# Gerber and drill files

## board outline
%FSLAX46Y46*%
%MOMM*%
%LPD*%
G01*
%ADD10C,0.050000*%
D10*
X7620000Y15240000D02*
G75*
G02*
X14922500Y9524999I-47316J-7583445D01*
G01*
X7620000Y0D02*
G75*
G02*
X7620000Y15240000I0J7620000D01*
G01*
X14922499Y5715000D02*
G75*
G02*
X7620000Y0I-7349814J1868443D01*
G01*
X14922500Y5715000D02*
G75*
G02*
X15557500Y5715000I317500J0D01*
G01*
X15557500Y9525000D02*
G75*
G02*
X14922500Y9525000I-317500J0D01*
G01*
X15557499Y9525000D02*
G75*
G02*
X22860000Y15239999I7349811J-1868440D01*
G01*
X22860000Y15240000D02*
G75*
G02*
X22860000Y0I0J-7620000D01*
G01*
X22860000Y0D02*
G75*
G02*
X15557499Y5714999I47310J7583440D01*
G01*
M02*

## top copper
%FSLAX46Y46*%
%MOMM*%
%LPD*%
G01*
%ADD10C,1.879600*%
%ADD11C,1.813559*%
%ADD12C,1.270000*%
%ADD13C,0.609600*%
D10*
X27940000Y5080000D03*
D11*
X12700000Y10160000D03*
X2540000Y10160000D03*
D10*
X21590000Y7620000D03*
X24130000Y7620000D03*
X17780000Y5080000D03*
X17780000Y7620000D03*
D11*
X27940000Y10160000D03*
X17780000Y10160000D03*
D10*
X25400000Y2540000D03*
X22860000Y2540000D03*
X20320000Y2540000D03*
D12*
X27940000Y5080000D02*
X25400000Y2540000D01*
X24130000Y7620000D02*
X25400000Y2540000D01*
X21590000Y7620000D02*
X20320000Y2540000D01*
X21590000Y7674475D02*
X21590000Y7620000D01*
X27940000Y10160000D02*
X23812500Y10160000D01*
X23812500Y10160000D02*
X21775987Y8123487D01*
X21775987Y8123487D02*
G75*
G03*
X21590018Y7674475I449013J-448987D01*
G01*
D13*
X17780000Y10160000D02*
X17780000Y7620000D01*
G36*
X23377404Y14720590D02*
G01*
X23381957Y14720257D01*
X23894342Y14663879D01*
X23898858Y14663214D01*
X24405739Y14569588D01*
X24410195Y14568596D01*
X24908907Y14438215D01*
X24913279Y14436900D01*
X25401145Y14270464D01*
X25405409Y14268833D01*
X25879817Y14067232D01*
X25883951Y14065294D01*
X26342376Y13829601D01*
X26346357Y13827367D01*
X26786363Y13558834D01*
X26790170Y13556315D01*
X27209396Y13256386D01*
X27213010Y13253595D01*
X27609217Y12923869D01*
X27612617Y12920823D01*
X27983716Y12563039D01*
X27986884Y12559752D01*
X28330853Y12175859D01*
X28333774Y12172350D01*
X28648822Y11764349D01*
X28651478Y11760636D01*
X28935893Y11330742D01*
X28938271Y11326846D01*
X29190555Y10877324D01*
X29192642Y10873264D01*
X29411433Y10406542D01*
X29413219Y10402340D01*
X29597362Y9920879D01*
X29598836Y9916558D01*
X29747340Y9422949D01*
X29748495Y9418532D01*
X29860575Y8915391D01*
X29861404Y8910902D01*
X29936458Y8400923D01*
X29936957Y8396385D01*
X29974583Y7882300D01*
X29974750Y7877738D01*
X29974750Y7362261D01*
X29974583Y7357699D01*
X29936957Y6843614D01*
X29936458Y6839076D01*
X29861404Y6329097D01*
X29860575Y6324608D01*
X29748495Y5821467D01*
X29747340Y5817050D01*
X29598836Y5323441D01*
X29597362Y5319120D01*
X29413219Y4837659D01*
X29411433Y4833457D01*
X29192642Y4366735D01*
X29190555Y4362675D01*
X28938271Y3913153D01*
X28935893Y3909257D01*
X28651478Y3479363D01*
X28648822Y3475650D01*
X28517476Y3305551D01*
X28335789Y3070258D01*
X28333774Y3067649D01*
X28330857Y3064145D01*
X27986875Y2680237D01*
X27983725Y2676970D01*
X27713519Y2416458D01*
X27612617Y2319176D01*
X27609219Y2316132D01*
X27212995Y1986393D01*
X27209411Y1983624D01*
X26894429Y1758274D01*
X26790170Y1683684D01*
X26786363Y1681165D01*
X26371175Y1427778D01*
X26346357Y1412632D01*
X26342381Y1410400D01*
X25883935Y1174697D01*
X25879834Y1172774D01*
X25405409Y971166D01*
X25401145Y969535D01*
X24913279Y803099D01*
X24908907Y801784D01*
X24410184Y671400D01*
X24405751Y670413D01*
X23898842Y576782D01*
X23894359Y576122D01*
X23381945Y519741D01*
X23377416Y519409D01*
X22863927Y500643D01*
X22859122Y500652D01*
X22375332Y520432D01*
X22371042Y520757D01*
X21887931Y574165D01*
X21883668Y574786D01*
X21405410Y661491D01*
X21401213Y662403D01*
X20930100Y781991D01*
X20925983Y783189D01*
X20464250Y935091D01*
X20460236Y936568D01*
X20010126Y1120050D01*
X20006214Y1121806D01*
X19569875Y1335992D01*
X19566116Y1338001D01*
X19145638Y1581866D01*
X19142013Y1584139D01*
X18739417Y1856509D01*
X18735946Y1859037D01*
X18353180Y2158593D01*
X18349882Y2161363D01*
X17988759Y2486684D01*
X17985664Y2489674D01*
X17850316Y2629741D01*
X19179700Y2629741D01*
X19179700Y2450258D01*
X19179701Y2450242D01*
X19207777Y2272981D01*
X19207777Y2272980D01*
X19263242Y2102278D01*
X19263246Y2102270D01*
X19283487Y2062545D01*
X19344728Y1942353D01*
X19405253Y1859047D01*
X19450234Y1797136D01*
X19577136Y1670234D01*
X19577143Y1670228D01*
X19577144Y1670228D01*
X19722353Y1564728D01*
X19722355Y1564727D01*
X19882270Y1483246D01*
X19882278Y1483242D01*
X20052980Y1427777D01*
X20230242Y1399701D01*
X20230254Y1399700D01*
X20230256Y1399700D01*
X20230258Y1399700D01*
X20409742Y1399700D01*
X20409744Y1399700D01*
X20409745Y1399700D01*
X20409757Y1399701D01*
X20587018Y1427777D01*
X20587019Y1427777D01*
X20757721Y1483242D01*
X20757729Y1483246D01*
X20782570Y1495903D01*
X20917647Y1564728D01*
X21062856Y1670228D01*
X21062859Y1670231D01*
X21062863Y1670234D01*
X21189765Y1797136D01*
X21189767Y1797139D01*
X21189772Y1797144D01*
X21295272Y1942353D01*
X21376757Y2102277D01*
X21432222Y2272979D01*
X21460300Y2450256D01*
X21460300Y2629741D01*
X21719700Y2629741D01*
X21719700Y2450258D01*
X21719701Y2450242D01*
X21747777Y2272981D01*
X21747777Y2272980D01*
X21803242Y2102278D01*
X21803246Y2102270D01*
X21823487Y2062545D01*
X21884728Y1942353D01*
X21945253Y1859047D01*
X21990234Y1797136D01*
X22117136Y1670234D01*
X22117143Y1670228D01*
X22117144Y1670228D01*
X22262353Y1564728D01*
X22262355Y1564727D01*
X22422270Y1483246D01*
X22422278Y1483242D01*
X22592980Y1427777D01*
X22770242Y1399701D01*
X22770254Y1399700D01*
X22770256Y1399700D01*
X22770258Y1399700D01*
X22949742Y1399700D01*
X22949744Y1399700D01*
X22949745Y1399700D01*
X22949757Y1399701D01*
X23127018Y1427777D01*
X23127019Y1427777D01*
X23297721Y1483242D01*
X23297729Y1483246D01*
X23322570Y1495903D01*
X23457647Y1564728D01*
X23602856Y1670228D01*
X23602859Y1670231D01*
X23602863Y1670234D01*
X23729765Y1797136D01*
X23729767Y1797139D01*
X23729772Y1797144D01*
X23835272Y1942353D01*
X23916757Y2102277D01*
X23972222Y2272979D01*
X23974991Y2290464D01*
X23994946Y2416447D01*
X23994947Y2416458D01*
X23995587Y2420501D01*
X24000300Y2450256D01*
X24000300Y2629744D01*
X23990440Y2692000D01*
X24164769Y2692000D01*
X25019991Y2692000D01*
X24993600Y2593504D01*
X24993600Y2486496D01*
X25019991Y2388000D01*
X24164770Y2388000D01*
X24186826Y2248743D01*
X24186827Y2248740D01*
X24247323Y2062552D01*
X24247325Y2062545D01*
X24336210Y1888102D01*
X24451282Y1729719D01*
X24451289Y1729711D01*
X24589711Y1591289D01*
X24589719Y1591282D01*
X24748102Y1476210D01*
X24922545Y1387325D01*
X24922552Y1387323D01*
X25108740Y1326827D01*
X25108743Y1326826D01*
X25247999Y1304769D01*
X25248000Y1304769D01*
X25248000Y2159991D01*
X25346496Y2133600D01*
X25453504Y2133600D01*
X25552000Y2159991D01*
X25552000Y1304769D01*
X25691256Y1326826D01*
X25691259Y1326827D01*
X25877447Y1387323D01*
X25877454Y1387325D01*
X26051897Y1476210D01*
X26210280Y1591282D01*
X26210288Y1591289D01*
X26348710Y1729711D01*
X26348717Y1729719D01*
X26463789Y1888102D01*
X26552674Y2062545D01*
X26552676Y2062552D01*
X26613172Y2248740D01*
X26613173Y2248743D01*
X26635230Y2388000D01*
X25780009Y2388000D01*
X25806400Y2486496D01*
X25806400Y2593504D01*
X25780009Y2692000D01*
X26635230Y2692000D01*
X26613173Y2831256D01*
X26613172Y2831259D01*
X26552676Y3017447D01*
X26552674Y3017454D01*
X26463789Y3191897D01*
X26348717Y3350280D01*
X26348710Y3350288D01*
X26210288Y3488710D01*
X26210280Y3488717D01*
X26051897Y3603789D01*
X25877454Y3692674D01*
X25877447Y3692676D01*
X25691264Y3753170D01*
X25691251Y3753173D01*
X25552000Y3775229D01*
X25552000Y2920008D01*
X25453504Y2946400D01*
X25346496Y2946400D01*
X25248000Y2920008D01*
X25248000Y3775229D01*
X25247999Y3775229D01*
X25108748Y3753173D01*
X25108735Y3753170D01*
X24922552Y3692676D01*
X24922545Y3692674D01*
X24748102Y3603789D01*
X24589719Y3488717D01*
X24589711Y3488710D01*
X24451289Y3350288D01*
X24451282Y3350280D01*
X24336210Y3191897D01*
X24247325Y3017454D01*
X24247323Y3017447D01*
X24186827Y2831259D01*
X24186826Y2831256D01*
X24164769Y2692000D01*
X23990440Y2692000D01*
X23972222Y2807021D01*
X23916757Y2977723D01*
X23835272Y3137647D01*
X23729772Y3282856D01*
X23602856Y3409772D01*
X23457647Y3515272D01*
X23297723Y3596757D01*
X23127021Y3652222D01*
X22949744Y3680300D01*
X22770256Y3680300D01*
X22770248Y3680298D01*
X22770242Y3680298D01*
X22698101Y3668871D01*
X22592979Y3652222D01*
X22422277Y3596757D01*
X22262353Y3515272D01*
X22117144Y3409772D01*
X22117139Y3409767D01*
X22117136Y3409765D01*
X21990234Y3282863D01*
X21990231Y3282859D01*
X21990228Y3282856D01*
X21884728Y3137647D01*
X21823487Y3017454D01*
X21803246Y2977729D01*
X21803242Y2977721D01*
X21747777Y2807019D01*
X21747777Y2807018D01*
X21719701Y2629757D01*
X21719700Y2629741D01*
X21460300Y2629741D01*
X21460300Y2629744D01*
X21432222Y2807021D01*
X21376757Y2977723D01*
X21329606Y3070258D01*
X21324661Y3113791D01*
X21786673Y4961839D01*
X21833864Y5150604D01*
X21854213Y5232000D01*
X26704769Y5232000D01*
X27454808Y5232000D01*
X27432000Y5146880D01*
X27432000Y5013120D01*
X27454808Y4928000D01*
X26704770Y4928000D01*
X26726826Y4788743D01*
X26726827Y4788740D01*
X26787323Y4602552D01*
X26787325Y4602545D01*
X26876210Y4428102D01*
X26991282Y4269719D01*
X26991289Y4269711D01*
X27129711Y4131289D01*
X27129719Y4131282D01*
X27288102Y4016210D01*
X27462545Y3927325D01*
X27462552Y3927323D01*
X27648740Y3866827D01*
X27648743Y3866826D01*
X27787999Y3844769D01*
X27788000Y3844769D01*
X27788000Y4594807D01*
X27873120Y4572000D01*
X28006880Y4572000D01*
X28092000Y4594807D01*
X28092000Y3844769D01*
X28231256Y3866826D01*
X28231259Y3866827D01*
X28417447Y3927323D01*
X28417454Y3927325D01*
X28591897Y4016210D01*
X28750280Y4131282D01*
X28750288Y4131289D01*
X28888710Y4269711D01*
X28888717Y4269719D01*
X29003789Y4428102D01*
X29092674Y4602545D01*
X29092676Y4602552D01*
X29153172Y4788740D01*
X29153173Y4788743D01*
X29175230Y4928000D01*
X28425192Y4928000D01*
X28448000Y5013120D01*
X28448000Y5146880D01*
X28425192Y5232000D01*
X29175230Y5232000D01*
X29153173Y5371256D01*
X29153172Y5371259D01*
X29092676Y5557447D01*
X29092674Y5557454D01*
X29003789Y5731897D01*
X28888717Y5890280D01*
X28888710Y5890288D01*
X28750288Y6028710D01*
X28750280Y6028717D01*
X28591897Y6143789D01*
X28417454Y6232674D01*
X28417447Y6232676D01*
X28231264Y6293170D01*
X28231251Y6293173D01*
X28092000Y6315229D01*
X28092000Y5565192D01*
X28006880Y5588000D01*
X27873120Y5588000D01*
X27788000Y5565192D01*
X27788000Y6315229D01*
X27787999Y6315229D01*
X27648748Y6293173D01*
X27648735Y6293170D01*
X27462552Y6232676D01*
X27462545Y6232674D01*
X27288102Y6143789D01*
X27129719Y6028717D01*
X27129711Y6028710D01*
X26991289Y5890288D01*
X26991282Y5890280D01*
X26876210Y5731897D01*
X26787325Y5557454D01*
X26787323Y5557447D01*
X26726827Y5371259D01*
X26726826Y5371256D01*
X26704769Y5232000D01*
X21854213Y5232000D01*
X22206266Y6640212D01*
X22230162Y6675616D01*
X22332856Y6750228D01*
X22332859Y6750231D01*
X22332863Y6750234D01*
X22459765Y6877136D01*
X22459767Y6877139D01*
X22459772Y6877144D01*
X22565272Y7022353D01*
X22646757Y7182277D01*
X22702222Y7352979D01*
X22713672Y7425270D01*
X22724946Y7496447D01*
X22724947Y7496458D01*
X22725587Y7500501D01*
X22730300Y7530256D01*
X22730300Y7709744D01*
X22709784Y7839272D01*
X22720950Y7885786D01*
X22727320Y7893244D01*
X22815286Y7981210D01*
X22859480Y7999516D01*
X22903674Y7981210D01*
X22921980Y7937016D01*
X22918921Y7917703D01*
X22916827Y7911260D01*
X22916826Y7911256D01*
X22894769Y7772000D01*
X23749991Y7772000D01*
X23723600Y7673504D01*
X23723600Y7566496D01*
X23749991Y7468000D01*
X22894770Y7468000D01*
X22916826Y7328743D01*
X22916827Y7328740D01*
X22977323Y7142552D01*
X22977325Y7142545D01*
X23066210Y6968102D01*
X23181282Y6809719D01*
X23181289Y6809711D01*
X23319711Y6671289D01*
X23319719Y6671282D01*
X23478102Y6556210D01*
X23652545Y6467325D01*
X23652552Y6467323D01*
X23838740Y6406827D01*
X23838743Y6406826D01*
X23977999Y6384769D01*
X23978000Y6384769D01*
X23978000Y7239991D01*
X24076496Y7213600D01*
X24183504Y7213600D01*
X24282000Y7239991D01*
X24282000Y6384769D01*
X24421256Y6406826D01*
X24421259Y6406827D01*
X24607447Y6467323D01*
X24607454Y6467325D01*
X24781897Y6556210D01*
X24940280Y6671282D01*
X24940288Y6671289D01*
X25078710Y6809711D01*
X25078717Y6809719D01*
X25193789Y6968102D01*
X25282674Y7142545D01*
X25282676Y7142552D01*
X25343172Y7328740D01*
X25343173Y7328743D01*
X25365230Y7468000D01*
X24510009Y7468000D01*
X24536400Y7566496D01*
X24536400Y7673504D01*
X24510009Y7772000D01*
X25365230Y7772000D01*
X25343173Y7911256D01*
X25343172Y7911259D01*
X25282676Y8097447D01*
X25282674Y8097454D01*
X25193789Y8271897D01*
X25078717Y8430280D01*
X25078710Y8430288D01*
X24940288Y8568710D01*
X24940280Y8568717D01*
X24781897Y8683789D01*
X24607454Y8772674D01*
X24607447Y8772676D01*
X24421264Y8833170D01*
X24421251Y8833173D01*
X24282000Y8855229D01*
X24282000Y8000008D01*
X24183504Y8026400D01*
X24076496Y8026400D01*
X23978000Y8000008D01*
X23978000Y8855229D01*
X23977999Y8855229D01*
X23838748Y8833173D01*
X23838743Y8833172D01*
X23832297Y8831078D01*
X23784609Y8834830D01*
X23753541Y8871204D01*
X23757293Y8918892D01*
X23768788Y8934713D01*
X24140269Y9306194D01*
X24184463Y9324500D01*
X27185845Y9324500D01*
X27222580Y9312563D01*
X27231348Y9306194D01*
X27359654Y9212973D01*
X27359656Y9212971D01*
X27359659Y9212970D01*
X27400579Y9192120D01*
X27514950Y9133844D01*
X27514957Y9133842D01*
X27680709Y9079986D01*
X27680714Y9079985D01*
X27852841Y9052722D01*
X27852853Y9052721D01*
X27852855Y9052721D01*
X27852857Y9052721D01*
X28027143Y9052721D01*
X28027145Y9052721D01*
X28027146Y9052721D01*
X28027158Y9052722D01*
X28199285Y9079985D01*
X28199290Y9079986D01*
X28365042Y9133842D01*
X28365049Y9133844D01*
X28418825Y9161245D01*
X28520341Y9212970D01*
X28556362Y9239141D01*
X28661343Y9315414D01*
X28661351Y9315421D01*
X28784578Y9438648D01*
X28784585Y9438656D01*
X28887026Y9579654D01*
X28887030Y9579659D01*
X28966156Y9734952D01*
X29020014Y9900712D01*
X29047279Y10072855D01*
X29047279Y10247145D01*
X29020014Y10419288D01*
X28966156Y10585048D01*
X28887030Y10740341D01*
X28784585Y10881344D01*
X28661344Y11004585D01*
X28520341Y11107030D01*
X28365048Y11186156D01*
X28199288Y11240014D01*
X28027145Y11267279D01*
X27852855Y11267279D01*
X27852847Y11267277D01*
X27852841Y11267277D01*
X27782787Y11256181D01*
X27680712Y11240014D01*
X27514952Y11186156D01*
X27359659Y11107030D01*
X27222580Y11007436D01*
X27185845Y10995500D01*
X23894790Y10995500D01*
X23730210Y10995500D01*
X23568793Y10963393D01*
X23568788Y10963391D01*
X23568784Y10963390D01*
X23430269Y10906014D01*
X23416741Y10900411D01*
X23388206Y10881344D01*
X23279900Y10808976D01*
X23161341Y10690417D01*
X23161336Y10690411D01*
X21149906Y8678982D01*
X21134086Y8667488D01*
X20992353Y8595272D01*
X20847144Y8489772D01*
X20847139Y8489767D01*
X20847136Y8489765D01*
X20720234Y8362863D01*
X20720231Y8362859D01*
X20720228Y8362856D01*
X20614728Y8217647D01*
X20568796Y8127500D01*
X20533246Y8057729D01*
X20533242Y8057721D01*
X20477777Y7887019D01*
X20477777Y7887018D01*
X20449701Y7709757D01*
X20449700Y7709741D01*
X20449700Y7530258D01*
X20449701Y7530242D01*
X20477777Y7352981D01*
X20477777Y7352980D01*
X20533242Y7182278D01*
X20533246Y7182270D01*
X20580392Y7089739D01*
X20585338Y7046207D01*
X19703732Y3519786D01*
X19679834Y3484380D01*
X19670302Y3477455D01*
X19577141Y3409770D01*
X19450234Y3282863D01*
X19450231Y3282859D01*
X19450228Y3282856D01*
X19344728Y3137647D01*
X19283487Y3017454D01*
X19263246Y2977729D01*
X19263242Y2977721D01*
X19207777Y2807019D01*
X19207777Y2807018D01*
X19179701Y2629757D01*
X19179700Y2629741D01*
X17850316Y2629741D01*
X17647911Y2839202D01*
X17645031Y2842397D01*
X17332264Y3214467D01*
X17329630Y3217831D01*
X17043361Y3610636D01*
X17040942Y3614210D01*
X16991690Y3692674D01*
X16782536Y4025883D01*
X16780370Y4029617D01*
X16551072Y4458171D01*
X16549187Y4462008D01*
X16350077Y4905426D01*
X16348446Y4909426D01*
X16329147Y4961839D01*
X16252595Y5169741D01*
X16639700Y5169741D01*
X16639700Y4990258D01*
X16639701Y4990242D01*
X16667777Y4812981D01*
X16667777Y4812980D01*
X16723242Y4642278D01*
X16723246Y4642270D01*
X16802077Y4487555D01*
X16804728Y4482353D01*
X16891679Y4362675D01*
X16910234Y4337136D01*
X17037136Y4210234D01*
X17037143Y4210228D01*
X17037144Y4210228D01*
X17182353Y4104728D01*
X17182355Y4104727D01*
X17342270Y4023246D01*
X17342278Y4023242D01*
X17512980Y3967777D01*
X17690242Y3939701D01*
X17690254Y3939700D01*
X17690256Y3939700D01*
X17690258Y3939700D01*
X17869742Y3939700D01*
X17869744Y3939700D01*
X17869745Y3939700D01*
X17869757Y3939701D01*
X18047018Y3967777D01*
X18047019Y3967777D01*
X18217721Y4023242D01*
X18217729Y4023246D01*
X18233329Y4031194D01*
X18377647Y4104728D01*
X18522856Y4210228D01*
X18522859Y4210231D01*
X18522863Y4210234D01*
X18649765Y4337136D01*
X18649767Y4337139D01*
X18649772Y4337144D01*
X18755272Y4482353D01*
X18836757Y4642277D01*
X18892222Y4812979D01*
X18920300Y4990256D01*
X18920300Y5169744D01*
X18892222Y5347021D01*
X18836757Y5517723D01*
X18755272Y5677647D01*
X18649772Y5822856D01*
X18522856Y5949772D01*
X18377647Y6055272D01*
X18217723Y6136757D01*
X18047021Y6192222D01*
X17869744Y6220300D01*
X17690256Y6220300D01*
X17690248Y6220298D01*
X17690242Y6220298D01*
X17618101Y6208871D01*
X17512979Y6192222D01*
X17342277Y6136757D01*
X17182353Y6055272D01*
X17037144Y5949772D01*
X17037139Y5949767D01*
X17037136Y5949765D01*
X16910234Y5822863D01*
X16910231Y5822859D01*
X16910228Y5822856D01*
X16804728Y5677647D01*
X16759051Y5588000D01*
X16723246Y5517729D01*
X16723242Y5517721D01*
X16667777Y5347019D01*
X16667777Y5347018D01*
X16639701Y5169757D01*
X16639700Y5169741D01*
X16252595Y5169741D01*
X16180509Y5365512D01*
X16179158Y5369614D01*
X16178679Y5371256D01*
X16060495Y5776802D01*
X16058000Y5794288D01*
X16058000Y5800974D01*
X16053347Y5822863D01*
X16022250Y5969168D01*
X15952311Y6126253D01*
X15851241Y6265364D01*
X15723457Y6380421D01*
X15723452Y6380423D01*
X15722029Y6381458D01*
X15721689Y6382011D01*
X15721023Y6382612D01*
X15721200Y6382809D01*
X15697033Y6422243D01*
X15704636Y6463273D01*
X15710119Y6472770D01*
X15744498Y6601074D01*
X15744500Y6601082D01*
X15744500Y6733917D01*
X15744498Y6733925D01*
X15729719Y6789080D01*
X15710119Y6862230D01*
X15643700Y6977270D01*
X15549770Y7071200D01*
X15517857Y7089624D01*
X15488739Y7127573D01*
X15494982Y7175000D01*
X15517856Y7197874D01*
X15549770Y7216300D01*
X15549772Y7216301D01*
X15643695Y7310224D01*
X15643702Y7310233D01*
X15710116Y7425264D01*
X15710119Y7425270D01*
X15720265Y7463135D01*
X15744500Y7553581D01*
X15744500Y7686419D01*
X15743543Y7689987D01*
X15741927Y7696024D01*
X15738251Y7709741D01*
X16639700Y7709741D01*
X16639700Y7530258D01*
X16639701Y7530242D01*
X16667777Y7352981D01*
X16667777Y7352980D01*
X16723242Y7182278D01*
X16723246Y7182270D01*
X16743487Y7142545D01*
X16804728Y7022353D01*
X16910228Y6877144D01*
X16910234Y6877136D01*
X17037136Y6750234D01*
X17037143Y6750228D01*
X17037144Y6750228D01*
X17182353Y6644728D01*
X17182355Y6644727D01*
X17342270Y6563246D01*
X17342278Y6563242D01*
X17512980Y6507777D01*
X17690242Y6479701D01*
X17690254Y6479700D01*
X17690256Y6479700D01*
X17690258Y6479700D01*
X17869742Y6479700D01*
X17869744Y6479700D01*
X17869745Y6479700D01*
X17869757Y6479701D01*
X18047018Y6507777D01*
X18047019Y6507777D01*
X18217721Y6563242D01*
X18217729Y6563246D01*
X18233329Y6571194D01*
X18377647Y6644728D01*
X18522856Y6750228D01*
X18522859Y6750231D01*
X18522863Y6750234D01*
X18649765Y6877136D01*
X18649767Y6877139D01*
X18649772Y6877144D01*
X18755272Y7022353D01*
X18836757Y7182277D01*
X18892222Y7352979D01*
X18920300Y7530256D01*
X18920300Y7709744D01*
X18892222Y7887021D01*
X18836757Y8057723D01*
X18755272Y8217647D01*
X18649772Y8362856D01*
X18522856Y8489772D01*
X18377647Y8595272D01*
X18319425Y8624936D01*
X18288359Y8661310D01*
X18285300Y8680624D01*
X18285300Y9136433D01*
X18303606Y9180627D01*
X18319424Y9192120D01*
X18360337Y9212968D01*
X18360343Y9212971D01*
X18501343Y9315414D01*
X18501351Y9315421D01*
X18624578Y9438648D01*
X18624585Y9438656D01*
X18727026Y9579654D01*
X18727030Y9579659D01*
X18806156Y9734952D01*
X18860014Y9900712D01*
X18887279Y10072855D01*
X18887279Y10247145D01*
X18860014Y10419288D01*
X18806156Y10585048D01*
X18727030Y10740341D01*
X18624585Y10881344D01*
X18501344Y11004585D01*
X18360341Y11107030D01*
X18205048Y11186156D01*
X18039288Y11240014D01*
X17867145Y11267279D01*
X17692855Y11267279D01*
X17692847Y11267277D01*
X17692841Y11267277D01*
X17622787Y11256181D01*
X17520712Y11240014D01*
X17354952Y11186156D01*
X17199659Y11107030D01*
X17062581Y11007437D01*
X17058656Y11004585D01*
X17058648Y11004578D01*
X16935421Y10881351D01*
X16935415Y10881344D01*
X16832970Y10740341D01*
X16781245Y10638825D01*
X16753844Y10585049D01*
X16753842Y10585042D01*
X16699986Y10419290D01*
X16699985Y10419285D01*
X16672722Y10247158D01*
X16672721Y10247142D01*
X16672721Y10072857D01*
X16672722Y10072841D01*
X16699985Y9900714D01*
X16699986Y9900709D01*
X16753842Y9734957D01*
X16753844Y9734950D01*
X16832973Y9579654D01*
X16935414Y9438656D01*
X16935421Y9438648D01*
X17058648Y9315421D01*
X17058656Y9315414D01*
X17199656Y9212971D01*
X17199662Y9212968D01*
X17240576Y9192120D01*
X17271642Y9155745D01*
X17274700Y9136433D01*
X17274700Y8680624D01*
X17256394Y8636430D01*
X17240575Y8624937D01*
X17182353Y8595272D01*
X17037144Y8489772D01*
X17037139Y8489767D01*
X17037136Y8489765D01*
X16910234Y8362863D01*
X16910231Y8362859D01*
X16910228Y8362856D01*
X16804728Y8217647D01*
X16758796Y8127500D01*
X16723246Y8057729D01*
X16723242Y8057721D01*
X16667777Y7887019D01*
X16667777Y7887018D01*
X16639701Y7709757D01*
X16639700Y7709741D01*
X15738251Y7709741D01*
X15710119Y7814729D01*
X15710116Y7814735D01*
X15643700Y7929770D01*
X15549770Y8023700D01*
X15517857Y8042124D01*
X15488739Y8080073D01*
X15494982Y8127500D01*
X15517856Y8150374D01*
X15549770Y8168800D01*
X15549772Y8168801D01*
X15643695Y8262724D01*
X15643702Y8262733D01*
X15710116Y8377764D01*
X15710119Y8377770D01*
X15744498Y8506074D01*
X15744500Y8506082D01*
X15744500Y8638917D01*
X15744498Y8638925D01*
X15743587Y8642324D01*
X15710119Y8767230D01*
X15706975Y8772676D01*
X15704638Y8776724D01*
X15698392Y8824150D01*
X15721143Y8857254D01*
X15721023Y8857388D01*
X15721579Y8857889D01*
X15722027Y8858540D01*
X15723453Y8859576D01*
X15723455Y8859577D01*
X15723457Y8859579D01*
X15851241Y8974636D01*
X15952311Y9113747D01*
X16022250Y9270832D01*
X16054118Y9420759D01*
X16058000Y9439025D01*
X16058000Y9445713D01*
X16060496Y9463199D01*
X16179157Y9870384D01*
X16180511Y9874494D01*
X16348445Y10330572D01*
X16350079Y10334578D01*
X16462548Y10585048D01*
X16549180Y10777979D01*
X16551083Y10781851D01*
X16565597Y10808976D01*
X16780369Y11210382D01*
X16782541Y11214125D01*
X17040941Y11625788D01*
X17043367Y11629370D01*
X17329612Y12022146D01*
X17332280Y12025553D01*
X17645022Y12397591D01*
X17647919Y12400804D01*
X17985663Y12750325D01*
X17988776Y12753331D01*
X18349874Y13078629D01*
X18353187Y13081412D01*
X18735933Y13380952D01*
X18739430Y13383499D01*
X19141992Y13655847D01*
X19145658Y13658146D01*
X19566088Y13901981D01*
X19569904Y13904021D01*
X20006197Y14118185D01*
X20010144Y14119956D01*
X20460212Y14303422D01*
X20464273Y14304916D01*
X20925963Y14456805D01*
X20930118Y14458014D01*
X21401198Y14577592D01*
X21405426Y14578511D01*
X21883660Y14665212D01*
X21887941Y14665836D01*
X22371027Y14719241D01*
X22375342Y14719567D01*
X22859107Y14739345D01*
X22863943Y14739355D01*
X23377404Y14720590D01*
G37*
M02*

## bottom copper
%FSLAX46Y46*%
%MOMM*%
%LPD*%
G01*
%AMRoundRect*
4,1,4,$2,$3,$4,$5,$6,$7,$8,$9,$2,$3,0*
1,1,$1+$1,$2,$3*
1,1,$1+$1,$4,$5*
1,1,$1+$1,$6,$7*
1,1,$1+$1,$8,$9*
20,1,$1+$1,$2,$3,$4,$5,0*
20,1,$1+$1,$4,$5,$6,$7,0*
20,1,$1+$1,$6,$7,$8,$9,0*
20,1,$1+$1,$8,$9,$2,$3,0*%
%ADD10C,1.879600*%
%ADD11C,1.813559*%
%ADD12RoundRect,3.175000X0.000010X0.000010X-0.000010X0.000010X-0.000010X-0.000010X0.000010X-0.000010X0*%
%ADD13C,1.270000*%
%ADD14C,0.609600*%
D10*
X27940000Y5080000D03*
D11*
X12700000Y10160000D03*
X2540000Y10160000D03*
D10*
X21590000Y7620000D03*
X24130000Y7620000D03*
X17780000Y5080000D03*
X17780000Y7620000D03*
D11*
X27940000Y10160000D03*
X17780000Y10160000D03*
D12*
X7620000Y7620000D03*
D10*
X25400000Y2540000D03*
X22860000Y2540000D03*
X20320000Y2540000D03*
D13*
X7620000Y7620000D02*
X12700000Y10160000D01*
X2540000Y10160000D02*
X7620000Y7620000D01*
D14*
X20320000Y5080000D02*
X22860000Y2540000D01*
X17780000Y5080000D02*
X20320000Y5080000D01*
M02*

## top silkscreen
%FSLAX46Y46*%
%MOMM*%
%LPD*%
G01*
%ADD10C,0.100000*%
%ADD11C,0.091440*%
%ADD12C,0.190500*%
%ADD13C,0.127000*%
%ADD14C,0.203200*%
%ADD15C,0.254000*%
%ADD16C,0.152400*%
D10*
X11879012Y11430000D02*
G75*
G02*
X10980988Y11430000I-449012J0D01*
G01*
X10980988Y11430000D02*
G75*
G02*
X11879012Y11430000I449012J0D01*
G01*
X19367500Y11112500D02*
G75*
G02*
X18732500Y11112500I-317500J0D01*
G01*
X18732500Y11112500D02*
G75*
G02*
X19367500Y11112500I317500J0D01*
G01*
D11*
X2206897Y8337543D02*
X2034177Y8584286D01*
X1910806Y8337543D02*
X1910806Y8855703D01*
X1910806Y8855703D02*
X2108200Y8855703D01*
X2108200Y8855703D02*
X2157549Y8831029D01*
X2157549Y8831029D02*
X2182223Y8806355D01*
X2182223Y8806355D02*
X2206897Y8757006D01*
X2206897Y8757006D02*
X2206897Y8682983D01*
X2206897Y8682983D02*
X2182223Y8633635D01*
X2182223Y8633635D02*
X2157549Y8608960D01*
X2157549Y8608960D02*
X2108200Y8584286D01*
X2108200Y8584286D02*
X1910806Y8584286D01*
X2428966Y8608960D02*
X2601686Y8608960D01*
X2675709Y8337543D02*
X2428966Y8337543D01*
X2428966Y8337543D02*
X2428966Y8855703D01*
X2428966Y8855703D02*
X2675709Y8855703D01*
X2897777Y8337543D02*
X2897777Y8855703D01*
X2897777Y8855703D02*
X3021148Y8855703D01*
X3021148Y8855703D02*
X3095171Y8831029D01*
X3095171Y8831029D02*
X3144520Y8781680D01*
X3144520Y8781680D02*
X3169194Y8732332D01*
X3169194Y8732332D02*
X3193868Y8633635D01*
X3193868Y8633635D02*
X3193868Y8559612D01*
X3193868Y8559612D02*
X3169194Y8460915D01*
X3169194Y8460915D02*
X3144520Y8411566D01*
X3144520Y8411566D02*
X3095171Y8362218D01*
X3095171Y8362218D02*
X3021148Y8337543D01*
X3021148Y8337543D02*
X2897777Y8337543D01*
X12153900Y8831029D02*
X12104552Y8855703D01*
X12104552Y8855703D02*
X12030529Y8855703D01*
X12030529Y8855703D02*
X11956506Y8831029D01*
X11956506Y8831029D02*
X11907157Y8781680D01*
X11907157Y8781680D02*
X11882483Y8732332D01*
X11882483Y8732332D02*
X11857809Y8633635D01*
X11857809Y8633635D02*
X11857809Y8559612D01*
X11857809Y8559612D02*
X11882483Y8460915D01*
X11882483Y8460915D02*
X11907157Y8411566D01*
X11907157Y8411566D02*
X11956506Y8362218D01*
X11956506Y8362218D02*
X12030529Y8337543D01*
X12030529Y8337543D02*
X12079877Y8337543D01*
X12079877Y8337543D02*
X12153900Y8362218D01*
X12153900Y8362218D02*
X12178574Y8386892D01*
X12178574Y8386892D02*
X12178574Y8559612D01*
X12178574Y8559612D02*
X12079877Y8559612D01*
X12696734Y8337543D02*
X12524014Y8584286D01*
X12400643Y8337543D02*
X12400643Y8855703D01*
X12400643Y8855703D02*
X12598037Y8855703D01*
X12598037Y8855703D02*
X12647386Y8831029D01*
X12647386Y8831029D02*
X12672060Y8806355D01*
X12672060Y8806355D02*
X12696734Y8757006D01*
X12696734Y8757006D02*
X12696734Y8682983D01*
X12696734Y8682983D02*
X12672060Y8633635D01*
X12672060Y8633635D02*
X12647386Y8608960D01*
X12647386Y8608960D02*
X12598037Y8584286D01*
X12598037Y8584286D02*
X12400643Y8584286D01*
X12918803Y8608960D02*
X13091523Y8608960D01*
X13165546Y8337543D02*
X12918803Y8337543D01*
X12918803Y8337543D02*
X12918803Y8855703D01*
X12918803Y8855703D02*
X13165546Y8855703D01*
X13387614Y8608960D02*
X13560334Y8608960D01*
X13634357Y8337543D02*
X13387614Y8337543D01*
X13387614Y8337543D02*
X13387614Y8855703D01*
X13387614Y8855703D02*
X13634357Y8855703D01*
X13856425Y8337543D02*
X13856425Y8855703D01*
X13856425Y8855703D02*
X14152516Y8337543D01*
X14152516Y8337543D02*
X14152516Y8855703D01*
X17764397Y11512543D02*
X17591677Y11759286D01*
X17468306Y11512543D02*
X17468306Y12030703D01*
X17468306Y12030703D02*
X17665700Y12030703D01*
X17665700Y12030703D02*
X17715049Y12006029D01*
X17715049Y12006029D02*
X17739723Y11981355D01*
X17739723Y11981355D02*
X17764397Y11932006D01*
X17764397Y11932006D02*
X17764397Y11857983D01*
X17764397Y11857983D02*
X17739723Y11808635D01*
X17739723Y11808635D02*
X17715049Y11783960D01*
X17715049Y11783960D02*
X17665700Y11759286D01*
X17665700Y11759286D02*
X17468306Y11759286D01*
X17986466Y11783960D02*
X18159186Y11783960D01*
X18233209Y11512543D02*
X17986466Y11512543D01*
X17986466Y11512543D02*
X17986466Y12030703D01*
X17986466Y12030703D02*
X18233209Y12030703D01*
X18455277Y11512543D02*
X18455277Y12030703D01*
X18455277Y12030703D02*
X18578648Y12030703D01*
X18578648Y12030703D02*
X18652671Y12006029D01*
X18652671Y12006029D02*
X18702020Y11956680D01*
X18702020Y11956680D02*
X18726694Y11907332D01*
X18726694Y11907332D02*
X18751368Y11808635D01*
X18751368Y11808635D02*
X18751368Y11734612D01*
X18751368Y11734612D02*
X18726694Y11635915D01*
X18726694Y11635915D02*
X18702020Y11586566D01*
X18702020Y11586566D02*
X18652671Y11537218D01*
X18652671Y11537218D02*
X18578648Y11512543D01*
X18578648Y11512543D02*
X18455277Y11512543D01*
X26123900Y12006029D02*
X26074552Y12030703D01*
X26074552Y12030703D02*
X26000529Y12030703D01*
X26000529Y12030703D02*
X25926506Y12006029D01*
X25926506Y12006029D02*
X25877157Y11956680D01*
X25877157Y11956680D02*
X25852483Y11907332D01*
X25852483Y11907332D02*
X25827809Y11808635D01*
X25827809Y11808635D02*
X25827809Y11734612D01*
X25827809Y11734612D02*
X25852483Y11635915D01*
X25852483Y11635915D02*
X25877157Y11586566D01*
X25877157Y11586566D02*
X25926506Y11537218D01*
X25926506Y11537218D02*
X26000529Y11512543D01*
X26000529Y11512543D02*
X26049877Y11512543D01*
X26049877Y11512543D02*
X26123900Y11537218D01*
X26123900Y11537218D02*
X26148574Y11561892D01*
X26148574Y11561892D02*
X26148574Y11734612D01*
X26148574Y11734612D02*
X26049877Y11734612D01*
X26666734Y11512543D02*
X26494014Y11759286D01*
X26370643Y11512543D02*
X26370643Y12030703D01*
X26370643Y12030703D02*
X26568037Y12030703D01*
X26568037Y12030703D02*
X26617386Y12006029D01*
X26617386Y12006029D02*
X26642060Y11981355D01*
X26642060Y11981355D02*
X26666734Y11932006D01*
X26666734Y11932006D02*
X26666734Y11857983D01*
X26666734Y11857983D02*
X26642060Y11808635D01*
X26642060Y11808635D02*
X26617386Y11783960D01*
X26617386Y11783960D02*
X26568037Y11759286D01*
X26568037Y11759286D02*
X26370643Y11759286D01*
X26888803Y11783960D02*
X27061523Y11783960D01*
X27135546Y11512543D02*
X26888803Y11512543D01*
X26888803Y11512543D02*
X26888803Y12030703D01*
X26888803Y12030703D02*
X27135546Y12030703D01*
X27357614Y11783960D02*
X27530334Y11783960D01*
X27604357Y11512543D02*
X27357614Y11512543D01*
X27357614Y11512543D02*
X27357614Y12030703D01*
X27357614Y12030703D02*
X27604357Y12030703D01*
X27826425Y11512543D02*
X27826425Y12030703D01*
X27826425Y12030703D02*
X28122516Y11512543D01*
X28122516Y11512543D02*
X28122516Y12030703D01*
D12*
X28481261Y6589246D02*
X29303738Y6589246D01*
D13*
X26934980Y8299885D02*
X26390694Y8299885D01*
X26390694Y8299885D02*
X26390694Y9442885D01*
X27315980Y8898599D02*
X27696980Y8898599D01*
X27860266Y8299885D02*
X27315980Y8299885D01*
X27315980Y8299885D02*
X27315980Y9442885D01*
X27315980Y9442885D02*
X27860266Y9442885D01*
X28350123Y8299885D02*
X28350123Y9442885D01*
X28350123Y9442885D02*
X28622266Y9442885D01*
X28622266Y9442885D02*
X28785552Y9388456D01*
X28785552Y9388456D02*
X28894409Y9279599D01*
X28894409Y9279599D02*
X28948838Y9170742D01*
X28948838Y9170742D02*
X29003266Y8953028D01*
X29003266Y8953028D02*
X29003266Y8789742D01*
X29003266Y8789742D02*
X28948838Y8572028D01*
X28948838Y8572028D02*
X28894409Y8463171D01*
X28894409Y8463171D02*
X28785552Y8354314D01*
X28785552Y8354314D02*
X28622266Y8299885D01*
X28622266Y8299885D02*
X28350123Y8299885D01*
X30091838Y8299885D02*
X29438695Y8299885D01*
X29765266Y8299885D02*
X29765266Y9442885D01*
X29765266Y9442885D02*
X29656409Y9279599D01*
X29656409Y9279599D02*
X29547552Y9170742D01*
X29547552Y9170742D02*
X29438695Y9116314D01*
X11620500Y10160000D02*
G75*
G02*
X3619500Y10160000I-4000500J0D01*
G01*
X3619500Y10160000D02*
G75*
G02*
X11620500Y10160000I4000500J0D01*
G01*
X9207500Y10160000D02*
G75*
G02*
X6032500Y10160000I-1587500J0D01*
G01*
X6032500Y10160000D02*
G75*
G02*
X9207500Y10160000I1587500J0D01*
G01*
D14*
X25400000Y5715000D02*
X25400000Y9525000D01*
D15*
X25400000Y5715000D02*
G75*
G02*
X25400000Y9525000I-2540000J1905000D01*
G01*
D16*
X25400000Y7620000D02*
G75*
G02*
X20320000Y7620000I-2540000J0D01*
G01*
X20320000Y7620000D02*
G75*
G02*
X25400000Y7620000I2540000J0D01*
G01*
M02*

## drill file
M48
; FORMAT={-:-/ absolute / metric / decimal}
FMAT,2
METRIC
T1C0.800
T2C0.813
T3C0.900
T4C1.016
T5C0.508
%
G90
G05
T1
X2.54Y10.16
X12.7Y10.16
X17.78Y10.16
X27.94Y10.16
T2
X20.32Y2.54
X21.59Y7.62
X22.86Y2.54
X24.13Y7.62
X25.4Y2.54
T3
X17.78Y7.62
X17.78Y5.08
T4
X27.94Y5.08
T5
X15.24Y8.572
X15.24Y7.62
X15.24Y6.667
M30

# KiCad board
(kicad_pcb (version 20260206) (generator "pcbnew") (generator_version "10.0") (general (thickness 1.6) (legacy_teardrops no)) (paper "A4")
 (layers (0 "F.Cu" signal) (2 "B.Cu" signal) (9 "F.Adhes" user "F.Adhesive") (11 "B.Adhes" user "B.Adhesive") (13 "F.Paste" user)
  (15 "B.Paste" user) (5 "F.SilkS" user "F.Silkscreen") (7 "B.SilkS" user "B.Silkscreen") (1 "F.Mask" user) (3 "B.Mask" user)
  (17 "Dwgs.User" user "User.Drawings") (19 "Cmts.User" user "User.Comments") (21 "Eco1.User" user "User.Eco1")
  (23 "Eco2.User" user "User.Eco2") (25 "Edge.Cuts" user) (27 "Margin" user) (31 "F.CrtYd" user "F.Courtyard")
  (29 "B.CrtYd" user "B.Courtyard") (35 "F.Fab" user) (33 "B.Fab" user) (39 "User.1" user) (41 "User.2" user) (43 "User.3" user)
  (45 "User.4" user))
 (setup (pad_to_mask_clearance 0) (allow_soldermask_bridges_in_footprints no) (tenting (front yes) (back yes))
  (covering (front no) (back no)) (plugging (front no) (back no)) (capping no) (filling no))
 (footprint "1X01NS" (layer "F.Cu") (at 27.94 -5.08)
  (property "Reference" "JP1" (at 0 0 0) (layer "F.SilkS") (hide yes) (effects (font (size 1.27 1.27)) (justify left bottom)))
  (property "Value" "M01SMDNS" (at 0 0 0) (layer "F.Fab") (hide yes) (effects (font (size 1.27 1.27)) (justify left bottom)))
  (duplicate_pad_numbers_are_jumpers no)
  (pad "1" thru_hole circle (at 0 0 90) (size 1.8796 1.8796) (drill 1.016) (layers "*.Cu" "*.Mask") (remove_unused_layers no) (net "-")
   (solder_mask_margin 0.0762) (thermal_bridge_angle 0)))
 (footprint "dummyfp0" (layer "F.Cu") (at 15.24 -7.62)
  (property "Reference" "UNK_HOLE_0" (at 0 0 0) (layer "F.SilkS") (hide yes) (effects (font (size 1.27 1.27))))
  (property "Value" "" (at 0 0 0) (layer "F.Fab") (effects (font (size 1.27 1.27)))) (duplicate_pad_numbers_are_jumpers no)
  (pad "" np_thru_hole circle (at 0 0) (size 0.508 0.508) (drill 0.508) (layers "*.Cu" "*.Mask")))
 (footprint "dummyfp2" (layer "F.Cu") (at 15.24 -8.5725)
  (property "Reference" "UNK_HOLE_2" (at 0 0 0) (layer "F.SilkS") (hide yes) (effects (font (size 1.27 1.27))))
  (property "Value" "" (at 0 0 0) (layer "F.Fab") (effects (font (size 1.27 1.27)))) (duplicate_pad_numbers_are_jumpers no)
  (pad "" np_thru_hole circle (at 0 0) (size 0.508 0.508) (drill 0.508) (layers "*.Cu" "*.Mask")))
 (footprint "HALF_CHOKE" (layer "F.Cu") (at 7.62 -10.16 180)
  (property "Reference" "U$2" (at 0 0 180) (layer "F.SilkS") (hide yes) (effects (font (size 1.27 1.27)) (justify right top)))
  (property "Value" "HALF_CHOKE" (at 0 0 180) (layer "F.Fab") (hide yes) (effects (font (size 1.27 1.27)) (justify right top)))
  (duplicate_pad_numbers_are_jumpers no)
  (fp_circle (center 0 0) (end 4.0005 0) (stroke (width 0.127) (type solid)) (fill no) (layer "F.SilkS"))
  (fp_circle (center 0 0) (end 1.5875 0) (stroke (width 0.127) (type solid)) (fill no) (layer "F.SilkS"))
  (pad "CENTER" thru_hole circle (at -5.08 0 180) (size 1.813559 1.813559) (drill 0.8) (layers "*.Cu" "*.Mask") (remove_unused_layers no)
   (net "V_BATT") (solder_mask_margin 0.0762) (thermal_bridge_angle 0))
  (pad "OUTSIDE" thru_hole circle (at 5.08 0 180) (size 1.813559 1.813559) (drill 0.8) (layers "*.Cu" "*.Mask") (remove_unused_layers no)
   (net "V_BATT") (solder_mask_margin 0.0762) (thermal_bridge_angle 0)))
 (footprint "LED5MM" (layer "F.Cu") (at 22.86 -7.62)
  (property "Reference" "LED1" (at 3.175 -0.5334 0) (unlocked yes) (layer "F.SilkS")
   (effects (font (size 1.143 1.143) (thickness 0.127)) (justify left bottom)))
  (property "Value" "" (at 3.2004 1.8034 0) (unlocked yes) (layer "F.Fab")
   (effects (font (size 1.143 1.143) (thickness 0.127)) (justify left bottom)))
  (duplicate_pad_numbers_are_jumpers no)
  (fp_line (start 2.54 1.905) (end 2.54 -1.905) (stroke (width 0.2032) (type solid)) (layer "F.SilkS"))
  (fp_arc (start 2.54 1.905) (mid -3.175 0) (end 2.54 -1.905) (stroke (width 0.254) (type solid)) (layer "F.SilkS"))
  (fp_circle (center 0 0) (end 2.54 0) (stroke (width 0.1524) (type solid)) (fill no) (layer "F.SilkS"))
  (pad "A" thru_hole circle (at -1.27 0) (size 1.8796 1.8796) (drill 0.8128) (layers "*.Cu" "*.Mask") (remove_unused_layers no) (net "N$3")
   (solder_mask_margin 0.0762) (thermal_bridge_angle 0))
  (pad "K" thru_hole circle (at 1.27 0) (size 1.8796 1.8796) (drill 0.8128) (layers "*.Cu" "*.Mask") (remove_unused_layers no) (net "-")
   (solder_mask_margin 0.0762) (thermal_bridge_angle 0)))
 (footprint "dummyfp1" (layer "F.Cu") (at 15.24 -6.6675)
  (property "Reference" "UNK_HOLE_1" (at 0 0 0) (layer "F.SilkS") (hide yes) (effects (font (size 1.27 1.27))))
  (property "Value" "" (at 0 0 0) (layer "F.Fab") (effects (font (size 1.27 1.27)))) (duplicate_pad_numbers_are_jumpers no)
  (pad "" np_thru_hole circle (at 0 0) (size 0.508 0.508) (drill 0.508) (layers "*.Cu" "*.Mask")))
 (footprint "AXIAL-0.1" (layer "B.Cu") (at 17.78 -5.08 90)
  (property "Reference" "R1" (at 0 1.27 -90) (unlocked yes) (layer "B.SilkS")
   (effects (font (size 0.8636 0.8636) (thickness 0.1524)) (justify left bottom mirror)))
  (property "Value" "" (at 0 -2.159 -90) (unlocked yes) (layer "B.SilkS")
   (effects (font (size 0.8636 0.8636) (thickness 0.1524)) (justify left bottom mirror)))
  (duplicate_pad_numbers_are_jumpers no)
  (pad "P$1" thru_hole circle (at 0 0 90) (size 1.8796 1.8796) (drill 0.9) (layers "*.Cu" "*.Mask") (remove_unused_layers no) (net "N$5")
   (solder_mask_margin 0.0762) (thermal_bridge_angle 0))
  (pad "P$2" thru_hole circle (at 2.54 0 90) (size 1.8796 1.8796) (drill 0.9) (layers "*.Cu" "*.Mask") (remove_unused_layers no) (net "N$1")
   (solder_mask_margin 0.0762) (thermal_bridge_angle 0)))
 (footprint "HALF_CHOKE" (layer "B.Cu") (at 22.86 -10.16 180)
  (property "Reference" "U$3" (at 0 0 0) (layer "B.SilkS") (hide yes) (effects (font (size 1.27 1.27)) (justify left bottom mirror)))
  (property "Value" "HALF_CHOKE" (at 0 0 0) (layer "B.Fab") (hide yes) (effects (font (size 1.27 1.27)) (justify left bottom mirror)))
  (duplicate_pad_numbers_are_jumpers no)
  (pad "CENTER" thru_hole circle (at -5.08 0 180) (size 1.813559 1.813559) (drill 0.8) (layers "*.Cu" "*.Mask") (remove_unused_layers no)
   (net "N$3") (solder_mask_margin 0.0762) (thermal_bridge_angle 0))
  (pad "OUTSIDE" thru_hole circle (at 5.08 0 180) (size 1.813559 1.813559) (drill 0.8) (layers "*.Cu" "*.Mask") (remove_unused_layers no)
   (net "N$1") (solder_mask_margin 0.0762) (thermal_bridge_angle 0)))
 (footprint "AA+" (layer "B.Cu") (at 7.62 -7.62 180)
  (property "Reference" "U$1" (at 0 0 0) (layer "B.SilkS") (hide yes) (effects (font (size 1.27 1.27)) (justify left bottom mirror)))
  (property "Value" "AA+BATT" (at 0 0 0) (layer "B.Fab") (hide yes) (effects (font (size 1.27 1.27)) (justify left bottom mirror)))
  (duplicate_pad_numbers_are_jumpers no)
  (pad "BATT+" smd roundrect (at 0 0 180) (size 6.35 6.35) (layers "B.Cu" "B.Mask" "B.Paste") (roundrect_rratio 0.5) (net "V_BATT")
   (solder_mask_margin 0.0762) (solder_paste_margin 0) (thermal_bridge_angle 0)))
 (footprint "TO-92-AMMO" (layer "B.Cu") (at 22.86 -2.54 180)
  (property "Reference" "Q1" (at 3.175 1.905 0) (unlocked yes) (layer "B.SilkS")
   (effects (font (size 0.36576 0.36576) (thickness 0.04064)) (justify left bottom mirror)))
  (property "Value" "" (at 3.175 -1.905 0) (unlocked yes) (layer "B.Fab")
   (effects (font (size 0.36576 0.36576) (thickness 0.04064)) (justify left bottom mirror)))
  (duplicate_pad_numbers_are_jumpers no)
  (pad "1" thru_hole circle (at -2.54 0 180) (size 1.8796 1.8796) (drill 0.8128) (layers "*.Cu" "*.Mask") (remove_unused_layers no)
   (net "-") (solder_mask_margin 0.0762) (thermal_bridge_angle 0))
  (pad "2" thru_hole circle (at 0 0 180) (size 1.8796 1.8796) (drill 0.8128) (layers "*.Cu" "*.Mask") (remove_unused_layers no) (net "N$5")
   (solder_mask_margin 0.0762) (thermal_bridge_angle 0))
  (pad "3" thru_hole circle (at 2.54 0 180) (size 1.8796 1.8796) (drill 0.8128) (layers "*.Cu" "*.Mask") (remove_unused_layers no)
   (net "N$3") (solder_mask_margin 0.0762) (thermal_bridge_angle 0)))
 (gr_circle (center 11.43 -11.43) (end 11.879012 -11.43) (stroke (width 0) (type solid)) (fill no) (layer "F.SilkS"))
 (gr_circle (center 19.05 -11.1125) (end 19.3675 -11.1125) (stroke (width 0) (type solid)) (fill no) (layer "F.SilkS"))
 (gr_arc (start 7.62 -15.24) (mid 12.246515 -13.628672) (end 14.9225 -9.524999) (stroke (width 0.05) (type solid)) (layer "Edge.Cuts"))
 (gr_arc (start 7.62 0) (mid 0 -7.62) (end 7.62 -15.24) (stroke (width 0.05) (type solid)) (layer "Edge.Cuts"))
 (gr_arc (start 14.922499 -5.715) (mid 12.246515 -1.611328) (end 7.62 0) (stroke (width 0.05) (type solid)) (layer "Edge.Cuts"))
 (gr_arc (start 14.9225 -5.715) (mid 15.24 -6.0325) (end 15.5575 -5.715) (stroke (width 0.05) (type solid)) (layer "Edge.Cuts"))
 (gr_arc (start 15.5575 -9.525) (mid 15.24 -9.2075) (end 14.9225 -9.525) (stroke (width 0.05) (type solid)) (layer "Edge.Cuts"))
 (gr_arc (start 15.557499 -9.525) (mid 18.233484 -13.628673) (end 22.86 -15.24) (stroke (width 0.05) (type solid)) (layer "Edge.Cuts"))
 (gr_arc (start 22.86 -15.24) (mid 30.48 -7.62) (end 22.86 0) (stroke (width 0.05) (type solid)) (layer "Edge.Cuts"))
 (gr_arc (start 22.86 0) (mid 18.233485 -1.611327) (end 15.5575 -5.714999) (stroke (width 0.05) (type solid)) (layer "Edge.Cuts"))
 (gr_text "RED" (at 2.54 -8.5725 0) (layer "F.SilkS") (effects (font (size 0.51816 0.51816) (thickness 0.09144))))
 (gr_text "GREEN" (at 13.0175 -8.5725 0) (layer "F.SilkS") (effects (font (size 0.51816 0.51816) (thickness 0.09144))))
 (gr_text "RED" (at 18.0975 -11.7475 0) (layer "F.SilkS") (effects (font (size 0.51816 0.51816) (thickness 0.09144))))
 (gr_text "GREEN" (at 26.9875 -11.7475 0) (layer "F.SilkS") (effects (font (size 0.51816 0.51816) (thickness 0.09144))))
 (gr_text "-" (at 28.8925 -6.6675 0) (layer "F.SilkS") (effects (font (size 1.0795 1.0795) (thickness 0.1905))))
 (segment (start 7.62 -7.62) (end 12.7 -10.16) (width 1.27) (layer "B.Cu") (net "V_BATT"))
 (segment (start 2.54 -10.16) (end 7.62 -7.62) (width 1.27) (layer "B.Cu") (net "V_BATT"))
 (segment (start 27.94 -5.08) (end 25.4 -2.54) (width 1.27) (layer "F.Cu") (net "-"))
 (segment (start 24.13 -7.62) (end 25.4 -2.54) (width 1.27) (layer "F.Cu") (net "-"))
 (segment (start 21.59 -7.62) (end 20.32 -2.54) (width 1.27) (layer "F.Cu") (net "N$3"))
 (segment (start 21.59 -7.674475) (end 21.59 -7.62) (width 1.27) (layer "F.Cu") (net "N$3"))
 (segment (start 27.94 -10.16) (end 23.8125 -10.16) (width 1.27) (layer "F.Cu") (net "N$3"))
 (segment (start 23.8125 -10.16) (end 21.775987 -8.123487) (width 1.27) (layer "F.Cu") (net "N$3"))
 (arc (start 21.775987 -8.123487) (mid 21.638336 -7.917479) (end 21.59 -7.674475) (width 1.27) (layer "F.Cu") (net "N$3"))
 (segment (start 20.32 -5.08) (end 22.86 -2.54) (width 0.6096) (layer "B.Cu") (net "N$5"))
 (segment (start 17.78 -5.08) (end 20.32 -5.08) (width 0.6096) (layer "B.Cu") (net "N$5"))
 (segment (start 17.78 -10.16) (end 17.78 -7.62) (width 0.6096) (layer "F.Cu") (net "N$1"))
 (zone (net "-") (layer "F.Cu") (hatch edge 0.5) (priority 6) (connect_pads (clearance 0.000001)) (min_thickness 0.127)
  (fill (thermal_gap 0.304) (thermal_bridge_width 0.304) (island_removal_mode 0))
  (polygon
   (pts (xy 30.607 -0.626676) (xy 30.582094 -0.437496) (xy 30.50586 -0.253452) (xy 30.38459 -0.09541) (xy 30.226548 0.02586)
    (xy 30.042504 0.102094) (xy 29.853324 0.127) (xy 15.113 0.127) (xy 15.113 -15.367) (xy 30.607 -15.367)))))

